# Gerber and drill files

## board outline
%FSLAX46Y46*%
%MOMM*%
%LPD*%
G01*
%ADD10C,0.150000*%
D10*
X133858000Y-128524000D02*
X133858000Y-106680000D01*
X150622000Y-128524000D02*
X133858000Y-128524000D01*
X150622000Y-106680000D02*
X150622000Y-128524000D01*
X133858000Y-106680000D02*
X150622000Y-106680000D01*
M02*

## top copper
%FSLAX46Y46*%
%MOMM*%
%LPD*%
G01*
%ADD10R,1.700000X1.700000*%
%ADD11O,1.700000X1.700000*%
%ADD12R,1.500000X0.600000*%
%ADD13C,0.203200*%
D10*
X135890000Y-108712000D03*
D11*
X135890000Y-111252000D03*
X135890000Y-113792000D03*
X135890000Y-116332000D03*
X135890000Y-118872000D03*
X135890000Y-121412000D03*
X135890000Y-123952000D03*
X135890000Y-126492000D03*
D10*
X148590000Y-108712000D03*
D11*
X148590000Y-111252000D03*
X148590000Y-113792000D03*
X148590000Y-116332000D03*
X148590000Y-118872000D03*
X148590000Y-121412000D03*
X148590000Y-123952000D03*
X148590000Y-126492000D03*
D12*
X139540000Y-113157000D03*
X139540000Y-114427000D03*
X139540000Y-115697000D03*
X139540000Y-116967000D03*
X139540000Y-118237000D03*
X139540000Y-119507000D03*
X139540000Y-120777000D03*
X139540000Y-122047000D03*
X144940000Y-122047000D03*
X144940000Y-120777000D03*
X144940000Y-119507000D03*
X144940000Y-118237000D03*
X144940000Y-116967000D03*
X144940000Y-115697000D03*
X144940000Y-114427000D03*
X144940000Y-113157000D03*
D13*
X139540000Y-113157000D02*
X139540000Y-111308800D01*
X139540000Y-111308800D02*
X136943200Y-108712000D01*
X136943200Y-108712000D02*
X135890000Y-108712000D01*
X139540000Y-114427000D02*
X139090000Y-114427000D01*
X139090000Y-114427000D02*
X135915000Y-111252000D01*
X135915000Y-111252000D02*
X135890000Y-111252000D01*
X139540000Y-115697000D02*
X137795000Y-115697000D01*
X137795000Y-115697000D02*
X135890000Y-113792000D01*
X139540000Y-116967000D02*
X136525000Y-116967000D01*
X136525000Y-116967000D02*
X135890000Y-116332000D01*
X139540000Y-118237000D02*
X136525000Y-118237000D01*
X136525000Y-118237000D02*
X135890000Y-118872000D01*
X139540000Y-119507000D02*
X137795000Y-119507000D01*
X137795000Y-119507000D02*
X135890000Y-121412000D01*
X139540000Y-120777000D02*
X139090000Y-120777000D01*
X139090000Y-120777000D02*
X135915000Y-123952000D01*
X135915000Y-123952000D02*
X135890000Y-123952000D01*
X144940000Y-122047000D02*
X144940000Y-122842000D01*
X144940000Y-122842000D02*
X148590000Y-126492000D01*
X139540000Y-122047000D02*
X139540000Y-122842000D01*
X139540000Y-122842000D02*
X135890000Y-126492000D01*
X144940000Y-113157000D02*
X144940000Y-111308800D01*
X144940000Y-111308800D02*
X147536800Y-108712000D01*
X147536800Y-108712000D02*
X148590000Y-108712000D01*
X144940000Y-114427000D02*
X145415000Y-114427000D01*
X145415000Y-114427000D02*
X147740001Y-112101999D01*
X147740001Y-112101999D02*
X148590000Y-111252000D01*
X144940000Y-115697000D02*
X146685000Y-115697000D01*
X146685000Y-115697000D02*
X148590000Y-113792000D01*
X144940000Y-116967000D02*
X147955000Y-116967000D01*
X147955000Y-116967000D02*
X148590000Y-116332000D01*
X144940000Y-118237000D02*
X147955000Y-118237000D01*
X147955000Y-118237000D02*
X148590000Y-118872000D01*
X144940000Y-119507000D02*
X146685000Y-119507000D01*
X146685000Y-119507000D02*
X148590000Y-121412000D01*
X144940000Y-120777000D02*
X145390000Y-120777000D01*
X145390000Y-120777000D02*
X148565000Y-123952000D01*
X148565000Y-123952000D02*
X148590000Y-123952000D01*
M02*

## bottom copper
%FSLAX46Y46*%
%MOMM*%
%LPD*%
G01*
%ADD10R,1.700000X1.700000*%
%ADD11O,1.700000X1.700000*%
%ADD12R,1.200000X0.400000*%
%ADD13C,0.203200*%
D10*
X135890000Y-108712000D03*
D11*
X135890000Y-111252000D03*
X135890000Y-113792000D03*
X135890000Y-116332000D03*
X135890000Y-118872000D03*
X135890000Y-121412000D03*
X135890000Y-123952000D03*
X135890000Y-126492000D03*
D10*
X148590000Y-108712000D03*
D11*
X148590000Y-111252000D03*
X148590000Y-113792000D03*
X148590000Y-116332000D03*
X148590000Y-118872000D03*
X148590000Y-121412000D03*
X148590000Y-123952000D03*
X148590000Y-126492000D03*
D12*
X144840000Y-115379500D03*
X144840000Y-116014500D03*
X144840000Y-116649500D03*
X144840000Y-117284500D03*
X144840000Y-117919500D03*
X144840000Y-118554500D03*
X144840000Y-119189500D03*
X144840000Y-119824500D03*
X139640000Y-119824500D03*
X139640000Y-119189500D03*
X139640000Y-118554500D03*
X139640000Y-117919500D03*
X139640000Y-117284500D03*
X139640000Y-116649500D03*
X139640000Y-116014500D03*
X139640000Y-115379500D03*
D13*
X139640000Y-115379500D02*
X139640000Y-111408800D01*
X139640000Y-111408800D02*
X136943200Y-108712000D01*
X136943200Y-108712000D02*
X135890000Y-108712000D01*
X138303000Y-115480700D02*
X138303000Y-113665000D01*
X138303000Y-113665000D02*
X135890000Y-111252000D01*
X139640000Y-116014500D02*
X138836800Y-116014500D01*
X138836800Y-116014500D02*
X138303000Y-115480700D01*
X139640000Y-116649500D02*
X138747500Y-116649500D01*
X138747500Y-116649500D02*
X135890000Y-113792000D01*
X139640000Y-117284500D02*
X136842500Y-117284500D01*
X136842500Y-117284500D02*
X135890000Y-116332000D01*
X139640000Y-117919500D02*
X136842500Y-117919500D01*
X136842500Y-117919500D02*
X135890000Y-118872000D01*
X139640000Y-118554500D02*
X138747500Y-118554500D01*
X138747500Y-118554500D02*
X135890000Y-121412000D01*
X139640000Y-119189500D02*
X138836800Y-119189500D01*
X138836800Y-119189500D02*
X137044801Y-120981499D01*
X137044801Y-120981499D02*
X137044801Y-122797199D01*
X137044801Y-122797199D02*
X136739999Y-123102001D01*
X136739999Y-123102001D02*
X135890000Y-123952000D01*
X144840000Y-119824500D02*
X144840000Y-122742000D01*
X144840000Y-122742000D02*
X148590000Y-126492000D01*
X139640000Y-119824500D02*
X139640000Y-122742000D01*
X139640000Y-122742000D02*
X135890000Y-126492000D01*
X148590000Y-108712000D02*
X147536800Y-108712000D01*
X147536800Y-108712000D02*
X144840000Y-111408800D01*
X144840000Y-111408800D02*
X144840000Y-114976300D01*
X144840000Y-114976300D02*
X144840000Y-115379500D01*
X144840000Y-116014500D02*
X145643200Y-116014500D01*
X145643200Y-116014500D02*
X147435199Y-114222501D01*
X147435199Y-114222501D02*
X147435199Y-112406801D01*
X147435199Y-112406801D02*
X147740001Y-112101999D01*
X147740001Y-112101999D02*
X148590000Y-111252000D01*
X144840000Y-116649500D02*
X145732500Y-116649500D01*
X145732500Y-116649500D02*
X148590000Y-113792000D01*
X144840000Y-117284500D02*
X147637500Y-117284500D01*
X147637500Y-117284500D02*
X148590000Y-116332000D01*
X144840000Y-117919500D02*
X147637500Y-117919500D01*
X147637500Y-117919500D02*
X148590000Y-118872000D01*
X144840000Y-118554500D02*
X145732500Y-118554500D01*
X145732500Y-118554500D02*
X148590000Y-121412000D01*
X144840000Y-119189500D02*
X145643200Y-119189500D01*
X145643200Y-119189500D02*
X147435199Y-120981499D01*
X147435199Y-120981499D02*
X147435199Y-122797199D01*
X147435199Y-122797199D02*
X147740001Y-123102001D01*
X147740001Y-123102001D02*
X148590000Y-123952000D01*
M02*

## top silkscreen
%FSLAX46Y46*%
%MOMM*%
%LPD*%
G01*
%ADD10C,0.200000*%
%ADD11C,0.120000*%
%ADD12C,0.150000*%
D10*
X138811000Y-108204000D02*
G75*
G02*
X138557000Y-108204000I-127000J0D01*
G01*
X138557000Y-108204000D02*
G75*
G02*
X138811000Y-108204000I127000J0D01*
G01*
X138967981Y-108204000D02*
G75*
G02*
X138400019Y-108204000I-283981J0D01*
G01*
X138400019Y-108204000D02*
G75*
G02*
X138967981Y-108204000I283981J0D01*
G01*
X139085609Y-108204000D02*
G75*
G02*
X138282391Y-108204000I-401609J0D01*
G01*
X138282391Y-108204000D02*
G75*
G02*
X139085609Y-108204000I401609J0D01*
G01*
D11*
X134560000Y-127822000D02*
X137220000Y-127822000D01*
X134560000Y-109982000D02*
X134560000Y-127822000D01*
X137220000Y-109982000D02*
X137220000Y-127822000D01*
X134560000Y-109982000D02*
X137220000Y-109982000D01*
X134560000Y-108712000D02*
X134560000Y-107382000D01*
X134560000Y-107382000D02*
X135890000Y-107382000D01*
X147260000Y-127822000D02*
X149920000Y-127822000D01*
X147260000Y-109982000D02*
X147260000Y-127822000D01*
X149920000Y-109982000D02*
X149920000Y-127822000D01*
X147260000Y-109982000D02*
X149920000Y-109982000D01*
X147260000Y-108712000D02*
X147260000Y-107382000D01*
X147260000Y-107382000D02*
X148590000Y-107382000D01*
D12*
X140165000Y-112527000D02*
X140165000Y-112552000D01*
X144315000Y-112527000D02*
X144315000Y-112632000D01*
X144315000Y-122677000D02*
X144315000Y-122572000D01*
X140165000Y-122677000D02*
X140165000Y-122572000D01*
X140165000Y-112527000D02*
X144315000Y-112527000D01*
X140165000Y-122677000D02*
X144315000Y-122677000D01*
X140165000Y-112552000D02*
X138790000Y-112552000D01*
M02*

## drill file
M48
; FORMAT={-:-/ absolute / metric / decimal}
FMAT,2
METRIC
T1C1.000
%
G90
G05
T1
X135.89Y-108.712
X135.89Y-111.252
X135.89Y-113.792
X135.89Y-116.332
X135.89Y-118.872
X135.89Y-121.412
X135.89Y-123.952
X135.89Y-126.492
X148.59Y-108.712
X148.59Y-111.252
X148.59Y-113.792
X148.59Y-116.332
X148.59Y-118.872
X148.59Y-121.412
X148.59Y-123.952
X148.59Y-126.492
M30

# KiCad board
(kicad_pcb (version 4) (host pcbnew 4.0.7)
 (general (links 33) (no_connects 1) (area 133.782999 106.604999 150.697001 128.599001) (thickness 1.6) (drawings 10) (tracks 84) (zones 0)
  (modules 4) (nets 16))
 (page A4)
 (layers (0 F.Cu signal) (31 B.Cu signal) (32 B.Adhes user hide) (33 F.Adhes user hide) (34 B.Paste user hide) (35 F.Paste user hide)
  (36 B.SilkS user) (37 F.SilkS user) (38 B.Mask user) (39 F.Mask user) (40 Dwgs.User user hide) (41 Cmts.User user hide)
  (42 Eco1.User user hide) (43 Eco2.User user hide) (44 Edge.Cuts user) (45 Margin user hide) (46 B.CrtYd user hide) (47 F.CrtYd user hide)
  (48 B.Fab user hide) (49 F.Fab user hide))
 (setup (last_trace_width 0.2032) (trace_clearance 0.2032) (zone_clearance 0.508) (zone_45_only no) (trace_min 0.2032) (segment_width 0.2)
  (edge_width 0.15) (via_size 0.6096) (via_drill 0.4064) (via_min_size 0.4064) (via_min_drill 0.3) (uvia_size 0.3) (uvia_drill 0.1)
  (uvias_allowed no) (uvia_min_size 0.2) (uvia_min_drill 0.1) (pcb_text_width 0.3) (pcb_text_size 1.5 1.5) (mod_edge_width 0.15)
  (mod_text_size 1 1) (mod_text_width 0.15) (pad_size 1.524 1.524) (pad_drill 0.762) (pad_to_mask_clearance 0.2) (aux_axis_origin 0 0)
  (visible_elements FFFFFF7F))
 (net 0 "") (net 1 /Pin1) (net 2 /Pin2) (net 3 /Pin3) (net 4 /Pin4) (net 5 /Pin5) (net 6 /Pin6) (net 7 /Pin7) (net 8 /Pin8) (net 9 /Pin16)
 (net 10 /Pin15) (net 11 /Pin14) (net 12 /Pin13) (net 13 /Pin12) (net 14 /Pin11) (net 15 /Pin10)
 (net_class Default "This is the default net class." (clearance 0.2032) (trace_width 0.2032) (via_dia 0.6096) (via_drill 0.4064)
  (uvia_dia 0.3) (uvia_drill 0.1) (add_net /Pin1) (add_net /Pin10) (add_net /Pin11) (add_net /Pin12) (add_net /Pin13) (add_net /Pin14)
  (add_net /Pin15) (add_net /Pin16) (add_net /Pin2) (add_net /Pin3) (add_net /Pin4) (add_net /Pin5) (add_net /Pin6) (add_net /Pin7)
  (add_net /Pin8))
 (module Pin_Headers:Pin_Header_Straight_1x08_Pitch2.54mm (layer F.Cu) (at 135.89 108.712)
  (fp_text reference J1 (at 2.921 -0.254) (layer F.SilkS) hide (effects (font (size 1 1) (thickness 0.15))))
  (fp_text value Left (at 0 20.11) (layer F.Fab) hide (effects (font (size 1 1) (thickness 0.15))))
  (fp_line (start -1.33 19.11) (end 1.33 19.11) (layer F.SilkS) (width 0.12))
  (fp_line (start -1.33 1.27) (end -1.33 19.11) (layer F.SilkS) (width 0.12))
  (fp_line (start 1.33 1.27) (end 1.33 19.11) (layer F.SilkS) (width 0.12))
  (fp_line (start -1.33 1.27) (end 1.33 1.27) (layer F.SilkS) (width 0.12))
  (fp_line (start -1.33 0) (end -1.33 -1.33) (layer F.SilkS) (width 0.12))
  (fp_line (start -1.33 -1.33) (end 0 -1.33) (layer F.SilkS) (width 0.12))
  (pad 1 thru_hole rect (at 0 0) (size 1.7 1.7) (drill 1) (layers *.Cu *.Mask) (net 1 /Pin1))
  (pad 2 thru_hole oval (at 0 2.54) (size 1.7 1.7) (drill 1) (layers *.Cu *.Mask) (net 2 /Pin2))
  (pad 3 thru_hole oval (at 0 5.08) (size 1.7 1.7) (drill 1) (layers *.Cu *.Mask) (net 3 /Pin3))
  (pad 4 thru_hole oval (at 0 7.62) (size 1.7 1.7) (drill 1) (layers *.Cu *.Mask) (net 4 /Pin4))
  (pad 5 thru_hole oval (at 0 10.16) (size 1.7 1.7) (drill 1) (layers *.Cu *.Mask) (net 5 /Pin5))
  (pad 6 thru_hole oval (at 0 12.7) (size 1.7 1.7) (drill 1) (layers *.Cu *.Mask) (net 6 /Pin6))
  (pad 7 thru_hole oval (at 0 15.24) (size 1.7 1.7) (drill 1) (layers *.Cu *.Mask) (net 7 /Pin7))
  (pad 8 thru_hole oval (at 0 17.78) (size 1.7 1.7) (drill 1) (layers *.Cu *.Mask) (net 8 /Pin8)))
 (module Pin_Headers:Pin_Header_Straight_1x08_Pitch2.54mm (layer F.Cu) (at 148.59 108.712)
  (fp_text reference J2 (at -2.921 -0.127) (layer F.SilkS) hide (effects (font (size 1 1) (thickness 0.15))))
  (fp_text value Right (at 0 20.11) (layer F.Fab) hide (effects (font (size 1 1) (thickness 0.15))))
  (fp_line (start -1.33 19.11) (end 1.33 19.11) (layer F.SilkS) (width 0.12))
  (fp_line (start -1.33 1.27) (end -1.33 19.11) (layer F.SilkS) (width 0.12))
  (fp_line (start 1.33 1.27) (end 1.33 19.11) (layer F.SilkS) (width 0.12))
  (fp_line (start -1.33 1.27) (end 1.33 1.27) (layer F.SilkS) (width 0.12))
  (fp_line (start -1.33 0) (end -1.33 -1.33) (layer F.SilkS) (width 0.12))
  (fp_line (start -1.33 -1.33) (end 0 -1.33) (layer F.SilkS) (width 0.12))
  (pad 1 thru_hole rect (at 0 0) (size 1.7 1.7) (drill 1) (layers *.Cu *.Mask) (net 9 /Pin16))
  (pad 2 thru_hole oval (at 0 2.54) (size 1.7 1.7) (drill 1) (layers *.Cu *.Mask) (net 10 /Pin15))
  (pad 3 thru_hole oval (at 0 5.08) (size 1.7 1.7) (drill 1) (layers *.Cu *.Mask) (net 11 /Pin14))
  (pad 4 thru_hole oval (at 0 7.62) (size 1.7 1.7) (drill 1) (layers *.Cu *.Mask) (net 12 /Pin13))
  (pad 5 thru_hole oval (at 0 10.16) (size 1.7 1.7) (drill 1) (layers *.Cu *.Mask) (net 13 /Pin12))
  (pad 6 thru_hole oval (at 0 12.7) (size 1.7 1.7) (drill 1) (layers *.Cu *.Mask) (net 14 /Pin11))
  (pad 7 thru_hole oval (at 0 15.24) (size 1.7 1.7) (drill 1) (layers *.Cu *.Mask) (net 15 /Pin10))
  (pad 8 thru_hole oval (at 0 17.78) (size 1.7 1.7) (drill 1) (layers *.Cu *.Mask) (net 8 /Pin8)))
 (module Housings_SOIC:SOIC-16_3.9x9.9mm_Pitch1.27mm (layer F.Cu) (at 142.24 117.602)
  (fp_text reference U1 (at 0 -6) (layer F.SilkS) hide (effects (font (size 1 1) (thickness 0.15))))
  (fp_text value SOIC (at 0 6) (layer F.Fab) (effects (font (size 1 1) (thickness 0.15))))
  (fp_line (start -2.075 -5.075) (end -2.075 -5.05) (layer F.SilkS) (width 0.15))
  (fp_line (start 2.075 -5.075) (end 2.075 -4.97) (layer F.SilkS) (width 0.15))
  (fp_line (start 2.075 5.075) (end 2.075 4.97) (layer F.SilkS) (width 0.15))
  (fp_line (start -2.075 5.075) (end -2.075 4.97) (layer F.SilkS) (width 0.15))
  (fp_line (start -2.075 -5.075) (end 2.075 -5.075) (layer F.SilkS) (width 0.15))
  (fp_line (start -2.075 5.075) (end 2.075 5.075) (layer F.SilkS) (width 0.15))
  (fp_line (start -2.075 -5.05) (end -3.45 -5.05) (layer F.SilkS) (width 0.15))
  (pad 1 smd rect (at -2.7 -4.445) (size 1.5 0.6) (layers F.Cu F.Paste F.Mask) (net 1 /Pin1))
  (pad 2 smd rect (at -2.7 -3.175) (size 1.5 0.6) (layers F.Cu F.Paste F.Mask) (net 2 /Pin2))
  (pad 3 smd rect (at -2.7 -1.905) (size 1.5 0.6) (layers F.Cu F.Paste F.Mask) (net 3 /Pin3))
  (pad 4 smd rect (at -2.7 -0.635) (size 1.5 0.6) (layers F.Cu F.Paste F.Mask) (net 4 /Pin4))
  (pad 5 smd rect (at -2.7 0.635) (size 1.5 0.6) (layers F.Cu F.Paste F.Mask) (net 5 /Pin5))
  (pad 6 smd rect (at -2.7 1.905) (size 1.5 0.6) (layers F.Cu F.Paste F.Mask) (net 6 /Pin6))
  (pad 7 smd rect (at -2.7 3.175) (size 1.5 0.6) (layers F.Cu F.Paste F.Mask) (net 7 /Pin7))
  (pad 8 smd rect (at -2.7 4.445) (size 1.5 0.6) (layers F.Cu F.Paste F.Mask) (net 8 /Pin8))
  (pad 9 smd rect (at 2.7 4.445) (size 1.5 0.6) (layers F.Cu F.Paste F.Mask) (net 8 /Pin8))
  (pad 10 smd rect (at 2.7 3.175) (size 1.5 0.6) (layers F.Cu F.Paste F.Mask) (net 15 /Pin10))
  (pad 11 smd rect (at 2.7 1.905) (size 1.5 0.6) (layers F.Cu F.Paste F.Mask) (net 14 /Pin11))
  (pad 12 smd rect (at 2.7 0.635) (size 1.5 0.6) (layers F.Cu F.Paste F.Mask) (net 13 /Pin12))
  (pad 13 smd rect (at 2.7 -0.635) (size 1.5 0.6) (layers F.Cu F.Paste F.Mask) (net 12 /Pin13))
  (pad 14 smd rect (at 2.7 -1.905) (size 1.5 0.6) (layers F.Cu F.Paste F.Mask) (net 11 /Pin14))
  (pad 15 smd rect (at 2.7 -3.175) (size 1.5 0.6) (layers F.Cu F.Paste F.Mask) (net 10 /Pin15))
  (pad 16 smd rect (at 2.7 -4.445) (size 1.5 0.6) (layers F.Cu F.Paste F.Mask) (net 9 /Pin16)))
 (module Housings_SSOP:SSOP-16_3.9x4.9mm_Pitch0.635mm (layer B.Cu) (at 142.24 117.602 180)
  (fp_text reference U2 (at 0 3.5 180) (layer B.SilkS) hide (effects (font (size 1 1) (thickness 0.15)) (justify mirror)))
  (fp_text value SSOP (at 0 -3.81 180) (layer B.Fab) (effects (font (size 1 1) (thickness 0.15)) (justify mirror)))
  (pad 1 smd rect (at -2.6 2.2225 180) (size 1.2 0.4) (layers B.Cu B.Paste B.Mask) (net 9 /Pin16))
  (pad 2 smd rect (at -2.6 1.5875 180) (size 1.2 0.4) (layers B.Cu B.Paste B.Mask) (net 10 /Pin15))
  (pad 3 smd rect (at -2.6 0.9525 180) (size 1.2 0.4) (layers B.Cu B.Paste B.Mask) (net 11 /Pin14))
  (pad 4 smd rect (at -2.6 0.3175 180) (size 1.2 0.4) (layers B.Cu B.Paste B.Mask) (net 12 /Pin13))
  (pad 5 smd rect (at -2.6 -0.3175 180) (size 1.2 0.4) (layers B.Cu B.Paste B.Mask) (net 13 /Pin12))
  (pad 6 smd rect (at -2.6 -0.9525 180) (size 1.2 0.4) (layers B.Cu B.Paste B.Mask) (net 14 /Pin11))
  (pad 7 smd rect (at -2.6 -1.5875 180) (size 1.2 0.4) (layers B.Cu B.Paste B.Mask) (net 15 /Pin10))
  (pad 8 smd rect (at -2.6 -2.2225 180) (size 1.2 0.4) (layers B.Cu B.Paste B.Mask) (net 8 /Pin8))
  (pad 9 smd rect (at 2.6 -2.2225 180) (size 1.2 0.4) (layers B.Cu B.Paste B.Mask) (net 8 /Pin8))
  (pad 10 smd rect (at 2.6 -1.5875 180) (size 1.2 0.4) (layers B.Cu B.Paste B.Mask) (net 7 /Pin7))
  (pad 11 smd rect (at 2.6 -0.9525 180) (size 1.2 0.4) (layers B.Cu B.Paste B.Mask) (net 6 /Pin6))
  (pad 12 smd rect (at 2.6 -0.3175 180) (size 1.2 0.4) (layers B.Cu B.Paste B.Mask) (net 5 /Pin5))
  (pad 13 smd rect (at 2.6 0.3175 180) (size 1.2 0.4) (layers B.Cu B.Paste B.Mask) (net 4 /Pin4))
  (pad 14 smd rect (at 2.6 0.9525 180) (size 1.2 0.4) (layers B.Cu B.Paste B.Mask) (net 3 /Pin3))
  (pad 15 smd rect (at 2.6 1.5875 180) (size 1.2 0.4) (layers B.Cu B.Paste B.Mask) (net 2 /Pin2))
  (pad 16 smd rect (at 2.6 2.2225 180) (size 1.2 0.4) (layers B.Cu B.Paste B.Mask) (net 1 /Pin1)))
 (gr_line (start 133.858 128.524) (end 133.858 106.68) (angle 90) (layer Edge.Cuts) (width 0.15))
 (gr_line (start 150.622 128.524) (end 133.858 128.524) (angle 90) (layer Edge.Cuts) (width 0.15))
 (gr_line (start 150.622 106.68) (end 150.622 128.524) (angle 90) (layer Edge.Cuts) (width 0.15))
 (gr_line (start 133.858 106.68) (end 150.622 106.68) (angle 90) (layer Edge.Cuts) (width 0.15))
 (gr_circle (center 138.684 108.204) (end 138.684 108.331) (layer F.SilkS) (width 0.2))
 (gr_circle (center 138.684 108.204) (end 138.811 108.458) (layer F.SilkS) (width 0.2))
 (gr_circle (center 138.684 108.204) (end 138.811 108.585) (layer F.SilkS) (width 0.2))
 (segment (start 139.64 115.3795) (end 139.64 111.4088) (width 0.2032) (layer B.Cu) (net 1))
 (segment (start 139.64 111.4088) (end 136.9432 108.712) (width 0.2032) (layer B.Cu) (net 1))
 (segment (start 136.9432 108.712) (end 135.89 108.712) (width 0.2032) (layer B.Cu) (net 1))
 (segment (start 139.54 113.157) (end 139.54 111.3088) (width 0.2032) (layer F.Cu) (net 1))
 (segment (start 139.54 111.3088) (end 136.9432 108.712) (width 0.2032) (layer F.Cu) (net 1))
 (segment (start 136.9432 108.712) (end 135.89 108.712) (width 0.2032) (layer F.Cu) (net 1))
 (segment (start 138.303 115.4807) (end 138.303 113.665) (width 0.2032) (layer B.Cu) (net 2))
 (segment (start 138.303 113.665) (end 135.89 111.252) (width 0.2032) (layer B.Cu) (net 2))
 (segment (start 139.64 116.0145) (end 138.8368 116.0145) (width 0.2032) (layer B.Cu) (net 2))
 (segment (start 138.8368 116.0145) (end 138.303 115.4807) (width 0.2032) (layer B.Cu) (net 2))
 (segment (start 139.54 114.427) (end 139.09 114.427) (width 0.2032) (layer F.Cu) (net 2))
 (segment (start 139.09 114.427) (end 135.915 111.252) (width 0.2032) (layer F.Cu) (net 2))
 (segment (start 135.915 111.252) (end 135.89 111.252) (width 0.2032) (layer F.Cu) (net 2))
 (segment (start 139.64 116.6495) (end 138.7475 116.6495) (width 0.2032) (layer B.Cu) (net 3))
 (segment (start 138.7475 116.6495) (end 135.89 113.792) (width 0.2032) (layer B.Cu) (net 3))
 (segment (start 139.54 115.697) (end 137.795 115.697) (width 0.2032) (layer F.Cu) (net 3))
 (segment (start 137.795 115.697) (end 135.89 113.792) (width 0.2032) (layer F.Cu) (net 3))
 (segment (start 139.64 117.2845) (end 136.8425 117.2845) (width 0.2032) (layer B.Cu) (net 4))
 (segment (start 136.8425 117.2845) (end 135.89 116.332) (width 0.2032) (layer B.Cu) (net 4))
 (segment (start 139.54 116.967) (end 136.525 116.967) (width 0.2032) (layer F.Cu) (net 4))
 (segment (start 136.525 116.967) (end 135.89 116.332) (width 0.2032) (layer F.Cu) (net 4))
 (segment (start 139.64 117.9195) (end 136.8425 117.9195) (width 0.2032) (layer B.Cu) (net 5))
 (segment (start 136.8425 117.9195) (end 135.89 118.872) (width 0.2032) (layer B.Cu) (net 5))
 (segment (start 139.54 118.237) (end 136.525 118.237) (width 0.2032) (layer F.Cu) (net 5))
 (segment (start 136.525 118.237) (end 135.89 118.872) (width 0.2032) (layer F.Cu) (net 5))
 (segment (start 139.64 118.5545) (end 138.7475 118.5545) (width 0.2032) (layer B.Cu) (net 6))
 (segment (start 138.7475 118.5545) (end 135.89 121.412) (width 0.2032) (layer B.Cu) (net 6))
 (segment (start 139.54 119.507) (end 137.795 119.507) (width 0.2032) (layer F.Cu) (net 6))
 (segment (start 137.795 119.507) (end 135.89 121.412) (width 0.2032) (layer F.Cu) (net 6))
 (segment (start 139.64 119.1895) (end 138.8368 119.1895) (width 0.2032) (layer B.Cu) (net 7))
 (segment (start 138.8368 119.1895) (end 137.044801 120.981499) (width 0.2032) (layer B.Cu) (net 7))
 (segment (start 137.044801 120.981499) (end 137.044801 122.797199) (width 0.2032) (layer B.Cu) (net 7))
 (segment (start 137.044801 122.797199) (end 136.739999 123.102001) (width 0.2032) (layer B.Cu) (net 7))
 (segment (start 136.739999 123.102001) (end 135.89 123.952) (width 0.2032) (layer B.Cu) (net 7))
 (segment (start 139.54 120.777) (end 139.09 120.777) (width 0.2032) (layer F.Cu) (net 7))
 (segment (start 139.09 120.777) (end 135.915 123.952) (width 0.2032) (layer F.Cu) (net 7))
 (segment (start 135.915 123.952) (end 135.89 123.952) (width 0.2032) (layer F.Cu) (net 7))
 (segment (start 144.84 119.8245) (end 144.84 122.742) (width 0.2032) (layer B.Cu) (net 8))
 (segment (start 144.84 122.742) (end 148.59 126.492) (width 0.2032) (layer B.Cu) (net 8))
 (segment (start 139.64 119.8245) (end 139.64 122.742) (width 0.2032) (layer B.Cu) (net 8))
 (segment (start 139.64 122.742) (end 135.89 126.492) (width 0.2032) (layer B.Cu) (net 8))
 (segment (start 144.94 122.047) (end 144.94 122.842) (width 0.2032) (layer F.Cu) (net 8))
 (segment (start 144.94 122.842) (end 148.59 126.492) (width 0.2032) (layer F.Cu) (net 8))
 (segment (start 139.54 122.047) (end 139.54 122.842) (width 0.2032) (layer F.Cu) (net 8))
 (segment (start 139.54 122.842) (end 135.89 126.492) (width 0.2032) (layer F.Cu) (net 8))
 (segment (start 148.59 108.712) (end 147.5368 108.712) (width 0.2032) (layer B.Cu) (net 9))
 (segment (start 147.5368 108.712) (end 144.84 111.4088) (width 0.2032) (layer B.Cu) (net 9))
 (segment (start 144.84 111.4088) (end 144.84 114.9763) (width 0.2032) (layer B.Cu) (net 9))
 (segment (start 144.84 114.9763) (end 144.84 115.3795) (width 0.2032) (layer B.Cu) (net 9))
 (segment (start 144.94 113.157) (end 144.94 111.3088) (width 0.2032) (layer F.Cu) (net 9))
 (segment (start 144.94 111.3088) (end 147.5368 108.712) (width 0.2032) (layer F.Cu) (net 9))
 (segment (start 147.5368 108.712) (end 148.59 108.712) (width 0.2032) (layer F.Cu) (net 9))
 (segment (start 144.84 116.0145) (end 145.6432 116.0145) (width 0.2032) (layer B.Cu) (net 10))
 (segment (start 145.6432 116.0145) (end 147.435199 114.222501) (width 0.2032) (layer B.Cu) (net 10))
 (segment (start 147.435199 114.222501) (end 147.435199 112.406801) (width 0.2032) (layer B.Cu) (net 10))
 (segment (start 147.435199 112.406801) (end 147.740001 112.101999) (width 0.2032) (layer B.Cu) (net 10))
 (segment (start 147.740001 112.101999) (end 148.59 111.252) (width 0.2032) (layer B.Cu) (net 10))
 (segment (start 144.94 114.427) (end 145.415 114.427) (width 0.2032) (layer F.Cu) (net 10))
 (segment (start 145.415 114.427) (end 147.740001 112.101999) (width 0.2032) (layer F.Cu) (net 10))
 (segment (start 147.740001 112.101999) (end 148.59 111.252) (width 0.2032) (layer F.Cu) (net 10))
 (segment (start 144.84 116.6495) (end 145.7325 116.6495) (width 0.2032) (layer B.Cu) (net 11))
 (segment (start 145.7325 116.6495) (end 148.59 113.792) (width 0.2032) (layer B.Cu) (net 11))
 (segment (start 144.94 115.697) (end 146.685 115.697) (width 0.2032) (layer F.Cu) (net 11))
 (segment (start 146.685 115.697) (end 148.59 113.792) (width 0.2032) (layer F.Cu) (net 11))
 (segment (start 144.84 117.2845) (end 147.6375 117.2845) (width 0.2032) (layer B.Cu) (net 12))
 (segment (start 147.6375 117.2845) (end 148.59 116.332) (width 0.2032) (layer B.Cu) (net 12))
 (segment (start 144.94 116.967) (end 147.955 116.967) (width 0.2032) (layer F.Cu) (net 12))
 (segment (start 147.955 116.967) (end 148.59 116.332) (width 0.2032) (layer F.Cu) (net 12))
 (segment (start 144.84 117.9195) (end 147.6375 117.9195) (width 0.2032) (layer B.Cu) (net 13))
 (segment (start 147.6375 117.9195) (end 148.59 118.872) (width 0.2032) (layer B.Cu) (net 13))
 (segment (start 144.94 118.237) (end 147.955 118.237) (width 0.2032) (layer F.Cu) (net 13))
 (segment (start 147.955 118.237) (end 148.59 118.872) (width 0.2032) (layer F.Cu) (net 13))
 (segment (start 144.84 118.5545) (end 145.7325 118.5545) (width 0.2032) (layer B.Cu) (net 14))
 (segment (start 145.7325 118.5545) (end 148.59 121.412) (width 0.2032) (layer B.Cu) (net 14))
 (segment (start 144.94 119.507) (end 146.685 119.507) (width 0.2032) (layer F.Cu) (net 14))
 (segment (start 146.685 119.507) (end 148.59 121.412) (width 0.2032) (layer F.Cu) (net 14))
 (segment (start 144.84 119.1895) (end 145.6432 119.1895) (width 0.2032) (layer B.Cu) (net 15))
 (segment (start 145.6432 119.1895) (end 147.435199 120.981499) (width 0.2032) (layer B.Cu) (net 15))
 (segment (start 147.435199 120.981499) (end 147.435199 122.797199) (width 0.2032) (layer B.Cu) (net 15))
 (segment (start 147.435199 122.797199) (end 147.740001 123.102001) (width 0.2032) (layer B.Cu) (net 15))
 (segment (start 147.740001 123.102001) (end 148.59 123.952) (width 0.2032) (layer B.Cu) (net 15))
 (segment (start 144.94 120.777) (end 145.39 120.777) (width 0.2032) (layer F.Cu) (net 15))
 (segment (start 145.39 120.777) (end 148.565 123.952) (width 0.2032) (layer F.Cu) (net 15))
 (segment (start 148.565 123.952) (end 148.59 123.952) (width 0.2032) (layer F.Cu) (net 15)))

